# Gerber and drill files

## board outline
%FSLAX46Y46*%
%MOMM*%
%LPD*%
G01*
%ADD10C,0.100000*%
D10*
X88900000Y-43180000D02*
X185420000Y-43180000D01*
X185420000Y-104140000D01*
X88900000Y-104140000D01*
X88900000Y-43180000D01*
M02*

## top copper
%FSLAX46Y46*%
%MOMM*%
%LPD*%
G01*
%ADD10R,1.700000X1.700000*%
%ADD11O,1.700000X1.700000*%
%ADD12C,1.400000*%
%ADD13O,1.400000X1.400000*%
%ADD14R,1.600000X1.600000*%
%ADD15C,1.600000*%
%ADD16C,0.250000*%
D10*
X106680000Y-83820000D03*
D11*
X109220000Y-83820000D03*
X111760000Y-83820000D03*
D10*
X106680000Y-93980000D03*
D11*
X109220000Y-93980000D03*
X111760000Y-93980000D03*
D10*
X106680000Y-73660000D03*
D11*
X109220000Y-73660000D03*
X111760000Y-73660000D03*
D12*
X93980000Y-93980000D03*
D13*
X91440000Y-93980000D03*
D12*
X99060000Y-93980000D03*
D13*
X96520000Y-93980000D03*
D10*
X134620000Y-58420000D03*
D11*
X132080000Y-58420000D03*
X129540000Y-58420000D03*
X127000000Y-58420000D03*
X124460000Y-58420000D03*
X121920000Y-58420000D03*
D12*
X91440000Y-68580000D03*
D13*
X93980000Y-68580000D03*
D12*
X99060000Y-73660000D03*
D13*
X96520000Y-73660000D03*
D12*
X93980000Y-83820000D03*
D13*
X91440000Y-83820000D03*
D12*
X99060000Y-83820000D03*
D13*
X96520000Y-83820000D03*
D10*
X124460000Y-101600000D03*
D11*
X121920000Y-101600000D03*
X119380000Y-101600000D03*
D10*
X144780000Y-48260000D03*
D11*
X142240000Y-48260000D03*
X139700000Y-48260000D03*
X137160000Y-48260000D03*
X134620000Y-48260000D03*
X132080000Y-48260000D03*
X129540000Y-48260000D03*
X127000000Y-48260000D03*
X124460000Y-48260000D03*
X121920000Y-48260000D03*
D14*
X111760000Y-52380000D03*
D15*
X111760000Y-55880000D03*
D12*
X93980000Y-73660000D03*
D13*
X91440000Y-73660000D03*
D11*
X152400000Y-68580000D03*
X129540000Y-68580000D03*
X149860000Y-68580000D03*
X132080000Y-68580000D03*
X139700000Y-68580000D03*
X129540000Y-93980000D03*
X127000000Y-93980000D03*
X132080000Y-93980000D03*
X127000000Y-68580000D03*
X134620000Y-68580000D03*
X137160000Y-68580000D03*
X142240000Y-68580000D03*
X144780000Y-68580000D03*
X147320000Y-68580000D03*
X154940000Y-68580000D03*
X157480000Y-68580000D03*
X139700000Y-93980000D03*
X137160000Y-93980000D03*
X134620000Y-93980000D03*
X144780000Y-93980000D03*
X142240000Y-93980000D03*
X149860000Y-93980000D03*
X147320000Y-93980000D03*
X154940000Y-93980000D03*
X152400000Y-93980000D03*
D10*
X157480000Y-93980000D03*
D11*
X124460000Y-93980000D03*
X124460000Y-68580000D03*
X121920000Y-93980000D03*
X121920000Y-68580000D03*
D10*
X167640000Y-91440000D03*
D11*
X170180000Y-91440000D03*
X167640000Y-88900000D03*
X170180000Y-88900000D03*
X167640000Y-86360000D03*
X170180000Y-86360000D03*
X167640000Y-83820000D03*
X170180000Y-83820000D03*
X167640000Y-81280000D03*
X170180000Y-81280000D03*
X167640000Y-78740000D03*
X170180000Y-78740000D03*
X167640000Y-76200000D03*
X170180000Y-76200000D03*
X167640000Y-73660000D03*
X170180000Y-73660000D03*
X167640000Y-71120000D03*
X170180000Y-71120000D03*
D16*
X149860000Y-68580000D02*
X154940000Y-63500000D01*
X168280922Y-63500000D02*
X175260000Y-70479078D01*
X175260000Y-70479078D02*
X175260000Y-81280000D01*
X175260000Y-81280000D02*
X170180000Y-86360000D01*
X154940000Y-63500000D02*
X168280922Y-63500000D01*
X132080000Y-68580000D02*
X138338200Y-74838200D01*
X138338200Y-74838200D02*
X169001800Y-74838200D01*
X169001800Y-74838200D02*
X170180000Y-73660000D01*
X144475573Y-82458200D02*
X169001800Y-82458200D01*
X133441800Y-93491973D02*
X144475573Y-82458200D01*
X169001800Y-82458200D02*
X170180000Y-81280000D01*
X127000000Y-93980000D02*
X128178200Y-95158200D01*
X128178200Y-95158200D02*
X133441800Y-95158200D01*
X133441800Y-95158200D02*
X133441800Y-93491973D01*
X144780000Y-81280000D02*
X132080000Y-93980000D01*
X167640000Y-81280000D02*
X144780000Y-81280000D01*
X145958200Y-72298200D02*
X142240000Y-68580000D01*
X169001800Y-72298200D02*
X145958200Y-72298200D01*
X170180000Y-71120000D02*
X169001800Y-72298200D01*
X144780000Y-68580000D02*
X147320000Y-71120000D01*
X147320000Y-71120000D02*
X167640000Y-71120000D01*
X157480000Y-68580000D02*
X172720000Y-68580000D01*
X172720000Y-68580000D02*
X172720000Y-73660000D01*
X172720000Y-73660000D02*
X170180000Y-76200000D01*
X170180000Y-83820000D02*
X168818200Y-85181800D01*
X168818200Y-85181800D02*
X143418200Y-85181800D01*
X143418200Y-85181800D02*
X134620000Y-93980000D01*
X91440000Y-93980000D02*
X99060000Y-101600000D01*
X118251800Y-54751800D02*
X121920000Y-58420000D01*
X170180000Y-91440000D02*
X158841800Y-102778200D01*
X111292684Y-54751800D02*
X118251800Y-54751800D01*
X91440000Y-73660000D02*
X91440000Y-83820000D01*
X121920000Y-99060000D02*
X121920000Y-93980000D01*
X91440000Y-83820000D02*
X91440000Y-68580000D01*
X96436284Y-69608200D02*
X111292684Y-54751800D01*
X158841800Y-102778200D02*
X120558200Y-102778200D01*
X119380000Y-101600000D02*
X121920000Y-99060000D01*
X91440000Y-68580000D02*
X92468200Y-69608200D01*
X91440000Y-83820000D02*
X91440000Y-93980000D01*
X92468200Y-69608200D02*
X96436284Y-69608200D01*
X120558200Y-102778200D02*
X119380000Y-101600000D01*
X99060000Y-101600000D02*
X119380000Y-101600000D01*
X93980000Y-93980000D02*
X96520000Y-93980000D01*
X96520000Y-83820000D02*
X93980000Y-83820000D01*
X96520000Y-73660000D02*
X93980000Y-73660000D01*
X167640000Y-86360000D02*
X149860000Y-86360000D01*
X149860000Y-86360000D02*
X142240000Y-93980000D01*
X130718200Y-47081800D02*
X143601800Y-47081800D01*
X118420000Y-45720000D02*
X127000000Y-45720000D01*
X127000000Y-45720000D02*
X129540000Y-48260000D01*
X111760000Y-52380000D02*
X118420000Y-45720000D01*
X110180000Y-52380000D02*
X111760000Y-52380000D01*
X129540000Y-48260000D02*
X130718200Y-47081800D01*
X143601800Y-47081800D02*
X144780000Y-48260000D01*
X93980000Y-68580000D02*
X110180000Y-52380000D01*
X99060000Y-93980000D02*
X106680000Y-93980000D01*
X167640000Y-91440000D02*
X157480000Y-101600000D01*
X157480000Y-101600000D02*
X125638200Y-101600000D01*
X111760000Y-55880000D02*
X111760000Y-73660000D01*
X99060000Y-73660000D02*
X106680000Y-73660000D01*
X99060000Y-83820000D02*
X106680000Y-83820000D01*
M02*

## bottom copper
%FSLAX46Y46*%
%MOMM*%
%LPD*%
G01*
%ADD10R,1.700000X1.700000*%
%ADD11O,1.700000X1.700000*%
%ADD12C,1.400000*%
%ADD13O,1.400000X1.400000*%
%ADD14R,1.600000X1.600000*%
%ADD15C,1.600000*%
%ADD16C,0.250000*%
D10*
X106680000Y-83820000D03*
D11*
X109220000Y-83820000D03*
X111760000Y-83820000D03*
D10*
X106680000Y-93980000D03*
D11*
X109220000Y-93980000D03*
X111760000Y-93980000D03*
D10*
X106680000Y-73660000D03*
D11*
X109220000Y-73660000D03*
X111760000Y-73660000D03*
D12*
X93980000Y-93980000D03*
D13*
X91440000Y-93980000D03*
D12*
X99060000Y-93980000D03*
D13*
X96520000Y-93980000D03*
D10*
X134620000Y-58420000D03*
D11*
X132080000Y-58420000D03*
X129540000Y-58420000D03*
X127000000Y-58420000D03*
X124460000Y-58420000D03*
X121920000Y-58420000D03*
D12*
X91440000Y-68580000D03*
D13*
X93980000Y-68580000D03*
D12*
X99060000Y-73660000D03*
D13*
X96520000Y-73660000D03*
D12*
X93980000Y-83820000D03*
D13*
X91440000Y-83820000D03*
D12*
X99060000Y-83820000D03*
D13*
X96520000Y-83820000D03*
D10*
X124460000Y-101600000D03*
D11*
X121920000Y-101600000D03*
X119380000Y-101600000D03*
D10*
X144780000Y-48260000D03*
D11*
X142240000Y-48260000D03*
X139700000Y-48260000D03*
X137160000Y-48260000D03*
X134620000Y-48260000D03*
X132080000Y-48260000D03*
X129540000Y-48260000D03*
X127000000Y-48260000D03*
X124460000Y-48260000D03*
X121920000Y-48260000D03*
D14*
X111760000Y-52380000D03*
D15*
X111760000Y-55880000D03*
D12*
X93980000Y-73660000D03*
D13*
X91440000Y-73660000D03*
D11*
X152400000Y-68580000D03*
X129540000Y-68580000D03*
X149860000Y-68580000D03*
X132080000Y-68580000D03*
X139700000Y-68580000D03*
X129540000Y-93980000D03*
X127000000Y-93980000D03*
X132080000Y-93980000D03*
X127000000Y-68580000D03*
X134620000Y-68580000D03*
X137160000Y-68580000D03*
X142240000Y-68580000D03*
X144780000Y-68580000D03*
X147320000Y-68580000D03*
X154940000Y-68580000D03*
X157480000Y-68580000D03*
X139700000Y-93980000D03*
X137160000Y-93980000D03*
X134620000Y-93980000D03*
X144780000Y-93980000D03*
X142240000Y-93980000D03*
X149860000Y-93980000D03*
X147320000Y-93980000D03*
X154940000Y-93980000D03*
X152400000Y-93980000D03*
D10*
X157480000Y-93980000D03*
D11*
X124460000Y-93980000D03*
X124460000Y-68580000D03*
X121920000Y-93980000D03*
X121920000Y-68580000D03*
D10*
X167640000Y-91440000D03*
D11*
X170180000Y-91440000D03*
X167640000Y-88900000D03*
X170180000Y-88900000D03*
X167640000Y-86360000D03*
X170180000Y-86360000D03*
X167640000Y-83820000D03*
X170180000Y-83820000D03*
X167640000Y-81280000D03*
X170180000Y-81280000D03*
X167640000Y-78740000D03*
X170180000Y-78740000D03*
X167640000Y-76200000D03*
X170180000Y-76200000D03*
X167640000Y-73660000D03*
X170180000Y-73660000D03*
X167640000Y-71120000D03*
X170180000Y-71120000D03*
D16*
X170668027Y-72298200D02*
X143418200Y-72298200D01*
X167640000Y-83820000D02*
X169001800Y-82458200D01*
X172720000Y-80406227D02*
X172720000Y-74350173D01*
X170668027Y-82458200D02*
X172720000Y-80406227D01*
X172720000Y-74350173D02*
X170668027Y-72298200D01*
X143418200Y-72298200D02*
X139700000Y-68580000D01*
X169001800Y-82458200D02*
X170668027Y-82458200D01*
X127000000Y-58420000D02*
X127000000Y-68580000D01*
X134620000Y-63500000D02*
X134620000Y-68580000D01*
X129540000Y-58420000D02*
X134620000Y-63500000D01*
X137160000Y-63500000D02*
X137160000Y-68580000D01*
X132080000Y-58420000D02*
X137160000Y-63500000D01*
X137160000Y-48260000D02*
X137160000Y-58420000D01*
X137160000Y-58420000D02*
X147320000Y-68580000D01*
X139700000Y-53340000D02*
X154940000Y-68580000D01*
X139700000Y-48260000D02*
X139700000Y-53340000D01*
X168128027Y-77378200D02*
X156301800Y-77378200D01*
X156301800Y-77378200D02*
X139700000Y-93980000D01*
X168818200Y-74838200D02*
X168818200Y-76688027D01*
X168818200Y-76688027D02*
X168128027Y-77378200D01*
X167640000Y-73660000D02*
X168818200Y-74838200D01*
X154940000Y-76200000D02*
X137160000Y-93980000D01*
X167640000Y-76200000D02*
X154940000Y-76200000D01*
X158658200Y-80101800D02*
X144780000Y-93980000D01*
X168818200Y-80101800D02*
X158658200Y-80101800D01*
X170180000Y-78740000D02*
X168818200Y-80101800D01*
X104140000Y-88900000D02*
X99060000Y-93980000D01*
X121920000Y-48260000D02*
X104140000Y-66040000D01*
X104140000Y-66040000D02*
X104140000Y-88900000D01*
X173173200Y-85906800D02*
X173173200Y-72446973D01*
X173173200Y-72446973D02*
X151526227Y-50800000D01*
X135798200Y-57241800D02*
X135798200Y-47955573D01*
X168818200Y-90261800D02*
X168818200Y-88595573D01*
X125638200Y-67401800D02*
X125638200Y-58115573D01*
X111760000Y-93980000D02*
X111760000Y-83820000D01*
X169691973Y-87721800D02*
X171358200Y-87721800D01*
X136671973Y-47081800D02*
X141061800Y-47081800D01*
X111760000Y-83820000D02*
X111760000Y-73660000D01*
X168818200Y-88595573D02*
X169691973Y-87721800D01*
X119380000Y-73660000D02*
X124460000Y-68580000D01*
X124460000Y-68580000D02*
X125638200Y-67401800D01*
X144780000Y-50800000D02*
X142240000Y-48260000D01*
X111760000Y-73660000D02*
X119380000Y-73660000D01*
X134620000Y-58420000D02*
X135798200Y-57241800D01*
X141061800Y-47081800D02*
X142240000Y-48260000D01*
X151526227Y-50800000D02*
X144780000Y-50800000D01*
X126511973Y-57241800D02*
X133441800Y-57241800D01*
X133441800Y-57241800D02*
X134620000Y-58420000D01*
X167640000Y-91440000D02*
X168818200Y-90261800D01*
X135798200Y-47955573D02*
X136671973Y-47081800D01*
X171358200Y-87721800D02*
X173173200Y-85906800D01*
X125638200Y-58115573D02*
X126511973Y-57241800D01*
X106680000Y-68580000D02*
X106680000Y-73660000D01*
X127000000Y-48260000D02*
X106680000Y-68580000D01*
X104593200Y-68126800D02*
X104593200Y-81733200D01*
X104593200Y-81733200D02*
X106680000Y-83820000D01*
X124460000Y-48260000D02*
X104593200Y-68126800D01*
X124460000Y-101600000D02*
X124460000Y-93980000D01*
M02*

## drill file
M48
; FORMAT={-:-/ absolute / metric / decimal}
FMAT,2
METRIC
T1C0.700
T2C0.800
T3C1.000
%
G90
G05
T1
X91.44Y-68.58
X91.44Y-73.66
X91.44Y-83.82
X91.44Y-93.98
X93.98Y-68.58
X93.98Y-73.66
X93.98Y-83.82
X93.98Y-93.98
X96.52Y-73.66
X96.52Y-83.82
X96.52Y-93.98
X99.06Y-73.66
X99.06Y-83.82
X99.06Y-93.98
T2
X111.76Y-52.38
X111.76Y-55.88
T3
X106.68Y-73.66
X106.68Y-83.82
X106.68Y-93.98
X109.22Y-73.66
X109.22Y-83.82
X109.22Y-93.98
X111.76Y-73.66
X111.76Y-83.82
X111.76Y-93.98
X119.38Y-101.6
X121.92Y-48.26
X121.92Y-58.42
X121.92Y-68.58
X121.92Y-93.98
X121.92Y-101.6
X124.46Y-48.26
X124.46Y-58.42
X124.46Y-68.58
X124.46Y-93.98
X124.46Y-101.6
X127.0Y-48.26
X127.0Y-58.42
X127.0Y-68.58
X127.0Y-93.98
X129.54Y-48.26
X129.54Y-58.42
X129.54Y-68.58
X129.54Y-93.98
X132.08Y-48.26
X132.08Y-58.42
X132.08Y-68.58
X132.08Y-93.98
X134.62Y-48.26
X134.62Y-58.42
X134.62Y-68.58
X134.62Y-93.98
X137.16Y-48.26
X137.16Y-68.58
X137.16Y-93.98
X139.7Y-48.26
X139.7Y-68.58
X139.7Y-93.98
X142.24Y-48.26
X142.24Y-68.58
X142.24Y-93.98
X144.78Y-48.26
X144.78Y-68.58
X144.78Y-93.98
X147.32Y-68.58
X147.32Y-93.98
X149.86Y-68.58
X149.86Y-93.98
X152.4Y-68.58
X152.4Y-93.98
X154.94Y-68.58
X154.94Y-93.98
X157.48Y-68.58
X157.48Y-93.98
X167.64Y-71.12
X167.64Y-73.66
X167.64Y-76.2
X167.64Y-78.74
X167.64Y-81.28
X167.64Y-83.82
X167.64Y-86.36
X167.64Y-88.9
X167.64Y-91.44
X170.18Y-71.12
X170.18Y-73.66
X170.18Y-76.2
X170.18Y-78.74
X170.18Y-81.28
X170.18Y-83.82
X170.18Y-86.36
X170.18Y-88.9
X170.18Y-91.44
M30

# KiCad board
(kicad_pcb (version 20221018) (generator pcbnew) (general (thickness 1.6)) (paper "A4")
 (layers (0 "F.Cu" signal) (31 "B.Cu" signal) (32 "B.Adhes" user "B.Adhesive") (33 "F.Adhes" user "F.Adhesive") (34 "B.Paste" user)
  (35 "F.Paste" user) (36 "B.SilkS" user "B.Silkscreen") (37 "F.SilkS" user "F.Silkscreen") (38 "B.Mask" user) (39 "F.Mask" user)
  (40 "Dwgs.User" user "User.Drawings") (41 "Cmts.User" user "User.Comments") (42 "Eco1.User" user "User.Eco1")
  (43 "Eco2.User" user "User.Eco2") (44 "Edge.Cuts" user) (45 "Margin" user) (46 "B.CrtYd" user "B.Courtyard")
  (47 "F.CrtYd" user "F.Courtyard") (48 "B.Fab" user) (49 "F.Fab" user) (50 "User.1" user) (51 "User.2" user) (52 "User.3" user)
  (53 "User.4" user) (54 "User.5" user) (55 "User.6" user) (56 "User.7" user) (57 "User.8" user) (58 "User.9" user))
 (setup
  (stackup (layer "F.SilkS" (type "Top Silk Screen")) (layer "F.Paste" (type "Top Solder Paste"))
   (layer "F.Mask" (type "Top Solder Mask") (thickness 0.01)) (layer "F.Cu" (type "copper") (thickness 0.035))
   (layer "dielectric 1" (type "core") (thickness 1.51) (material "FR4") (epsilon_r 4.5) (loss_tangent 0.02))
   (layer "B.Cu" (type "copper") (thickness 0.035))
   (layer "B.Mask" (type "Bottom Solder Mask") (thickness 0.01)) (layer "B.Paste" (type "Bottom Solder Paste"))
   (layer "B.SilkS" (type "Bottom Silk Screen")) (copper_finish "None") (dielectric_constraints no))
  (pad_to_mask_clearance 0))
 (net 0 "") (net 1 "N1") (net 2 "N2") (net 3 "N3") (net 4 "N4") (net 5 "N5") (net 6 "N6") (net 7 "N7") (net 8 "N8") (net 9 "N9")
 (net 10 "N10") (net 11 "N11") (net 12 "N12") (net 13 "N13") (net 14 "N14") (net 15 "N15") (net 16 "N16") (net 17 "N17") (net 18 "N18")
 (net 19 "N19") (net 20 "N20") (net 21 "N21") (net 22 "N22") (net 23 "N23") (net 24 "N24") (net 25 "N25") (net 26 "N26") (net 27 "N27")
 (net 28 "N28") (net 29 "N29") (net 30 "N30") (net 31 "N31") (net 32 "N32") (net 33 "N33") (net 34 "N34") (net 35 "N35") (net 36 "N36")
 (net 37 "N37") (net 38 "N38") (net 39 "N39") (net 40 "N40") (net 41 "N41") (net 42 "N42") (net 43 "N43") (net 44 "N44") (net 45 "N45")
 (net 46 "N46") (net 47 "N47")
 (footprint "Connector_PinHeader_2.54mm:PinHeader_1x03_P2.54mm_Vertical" (layer "F.Cu") (at 106.68 83.82 90)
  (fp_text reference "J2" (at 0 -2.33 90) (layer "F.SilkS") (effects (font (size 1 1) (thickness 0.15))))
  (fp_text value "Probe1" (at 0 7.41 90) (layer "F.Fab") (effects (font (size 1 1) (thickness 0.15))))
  (pad "1" thru_hole rect (at 0 0 90) (size 1.7 1.7) (drill 1) (layers "*.Cu" "*.Mask") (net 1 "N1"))
  (pad "2" thru_hole oval (at 0 2.54 90) (size 1.7 1.7) (drill 1) (layers "*.Cu" "*.Mask") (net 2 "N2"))
  (pad "3" thru_hole oval (at 0 5.08 90) (size 1.7 1.7) (drill 1) (layers "*.Cu" "*.Mask") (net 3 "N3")))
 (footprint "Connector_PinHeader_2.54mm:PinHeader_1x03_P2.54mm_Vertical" (layer "F.Cu") (at 106.68 93.98 90)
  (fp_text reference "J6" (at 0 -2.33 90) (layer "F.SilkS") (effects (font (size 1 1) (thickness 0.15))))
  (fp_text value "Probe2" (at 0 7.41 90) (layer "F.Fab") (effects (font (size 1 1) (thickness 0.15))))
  (pad "1" thru_hole rect (at 0 0 90) (size 1.7 1.7) (drill 1) (layers "*.Cu" "*.Mask") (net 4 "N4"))
  (pad "2" thru_hole oval (at 0 2.54 90) (size 1.7 1.7) (drill 1) (layers "*.Cu" "*.Mask") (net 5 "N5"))
  (pad "3" thru_hole oval (at 0 5.08 90) (size 1.7 1.7) (drill 1) (layers "*.Cu" "*.Mask") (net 3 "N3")))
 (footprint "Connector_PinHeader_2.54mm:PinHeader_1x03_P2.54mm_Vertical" (layer "F.Cu") (at 106.68 73.66 90)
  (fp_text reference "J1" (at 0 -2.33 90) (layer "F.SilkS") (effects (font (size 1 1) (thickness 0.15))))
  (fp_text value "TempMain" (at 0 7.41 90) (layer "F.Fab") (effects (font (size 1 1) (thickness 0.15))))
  (pad "1" thru_hole rect (at 0 0 90) (size 1.7 1.7) (drill 1) (layers "*.Cu" "*.Mask") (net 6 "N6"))
  (pad "2" thru_hole oval (at 0 2.54 90) (size 1.7 1.7) (drill 1) (layers "*.Cu" "*.Mask") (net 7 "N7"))
  (pad "3" thru_hole oval (at 0 5.08 90) (size 1.7 1.7) (drill 1) (layers "*.Cu" "*.Mask") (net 3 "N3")))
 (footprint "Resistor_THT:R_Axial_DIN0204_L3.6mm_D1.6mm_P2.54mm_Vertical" (layer "F.Cu") (at 93.98 93.98 180)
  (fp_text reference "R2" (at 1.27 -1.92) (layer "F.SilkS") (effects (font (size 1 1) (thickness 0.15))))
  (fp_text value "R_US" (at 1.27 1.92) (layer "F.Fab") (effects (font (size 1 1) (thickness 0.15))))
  (pad "1" thru_hole circle (at 0 0 180) (size 1.4 1.4) (drill 0.7) (layers "*.Cu" "*.Mask") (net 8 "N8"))
  (pad "2" thru_hole oval (at 2.54 0 180) (size 1.4 1.4) (drill 0.7) (layers "*.Cu" "*.Mask") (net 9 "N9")))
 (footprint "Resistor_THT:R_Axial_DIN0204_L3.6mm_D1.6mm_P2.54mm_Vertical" (layer "F.Cu") (at 99.06 93.98 180)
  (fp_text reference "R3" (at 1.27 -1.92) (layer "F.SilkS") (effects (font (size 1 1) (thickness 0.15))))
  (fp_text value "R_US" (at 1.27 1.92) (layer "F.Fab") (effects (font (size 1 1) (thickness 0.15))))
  (pad "1" thru_hole circle (at 0 0 180) (size 1.4 1.4) (drill 0.7) (layers "*.Cu" "*.Mask") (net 4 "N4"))
  (pad "2" thru_hole oval (at 2.54 0 180) (size 1.4 1.4) (drill 0.7) (layers "*.Cu" "*.Mask") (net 8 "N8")))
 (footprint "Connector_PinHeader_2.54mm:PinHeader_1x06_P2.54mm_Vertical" (layer "F.Cu") (at 134.62 58.42 -90)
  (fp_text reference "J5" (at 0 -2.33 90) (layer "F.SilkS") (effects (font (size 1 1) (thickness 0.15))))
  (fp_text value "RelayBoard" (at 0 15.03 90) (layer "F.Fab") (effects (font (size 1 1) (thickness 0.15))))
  (pad "1" thru_hole rect (at 0 0 270) (size 1.7 1.7) (drill 1) (layers "*.Cu" "*.Mask") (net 3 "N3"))
  (pad "2" thru_hole oval (at 0 2.54 270) (size 1.7 1.7) (drill 1) (layers "*.Cu" "*.Mask") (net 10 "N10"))
  (pad "3" thru_hole oval (at 0 5.08 270) (size 1.7 1.7) (drill 1) (layers "*.Cu" "*.Mask") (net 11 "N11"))
  (pad "4" thru_hole oval (at 0 7.62 270) (size 1.7 1.7) (drill 1) (layers "*.Cu" "*.Mask") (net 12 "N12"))
  (pad "5" thru_hole oval (at 0 10.16 270) (size 1.7 1.7) (drill 1) (layers "*.Cu" "*.Mask") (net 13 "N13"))
  (pad "6" thru_hole oval (at 0 12.7 270) (size 1.7 1.7) (drill 1) (layers "*.Cu" "*.Mask") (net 9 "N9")))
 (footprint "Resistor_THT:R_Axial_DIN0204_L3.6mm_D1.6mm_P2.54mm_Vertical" (layer "F.Cu") (at 91.44 68.58)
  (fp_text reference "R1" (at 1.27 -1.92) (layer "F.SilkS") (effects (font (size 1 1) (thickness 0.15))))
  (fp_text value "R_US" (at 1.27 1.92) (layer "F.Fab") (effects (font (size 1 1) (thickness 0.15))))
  (pad "1" thru_hole circle (at 0 0) (size 1.4 1.4) (drill 0.7) (layers "*.Cu" "*.Mask") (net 9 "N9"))
  (pad "2" thru_hole oval (at 2.54 0) (size 1.4 1.4) (drill 0.7) (layers "*.Cu" "*.Mask") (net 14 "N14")))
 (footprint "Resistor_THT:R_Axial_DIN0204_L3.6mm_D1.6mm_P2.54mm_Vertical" (layer "F.Cu") (at 99.06 73.66 180)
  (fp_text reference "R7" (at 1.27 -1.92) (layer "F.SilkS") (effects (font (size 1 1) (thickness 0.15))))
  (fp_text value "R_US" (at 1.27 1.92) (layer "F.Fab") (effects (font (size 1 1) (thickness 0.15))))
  (pad "1" thru_hole circle (at 0 0 180) (size 1.4 1.4) (drill 0.7) (layers "*.Cu" "*.Mask") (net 6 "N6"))
  (pad "2" thru_hole oval (at 2.54 0 180) (size 1.4 1.4) (drill 0.7) (layers "*.Cu" "*.Mask") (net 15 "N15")))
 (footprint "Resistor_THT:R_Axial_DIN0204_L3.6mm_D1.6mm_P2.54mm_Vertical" (layer "F.Cu") (at 93.98 83.82 180)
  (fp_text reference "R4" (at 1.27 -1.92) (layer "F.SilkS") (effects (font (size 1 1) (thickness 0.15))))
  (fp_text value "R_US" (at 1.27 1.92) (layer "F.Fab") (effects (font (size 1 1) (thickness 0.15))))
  (pad "1" thru_hole circle (at 0 0 180) (size 1.4 1.4) (drill 0.7) (layers "*.Cu" "*.Mask") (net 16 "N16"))
  (pad "2" thru_hole oval (at 2.54 0 180) (size 1.4 1.4) (drill 0.7) (layers "*.Cu" "*.Mask") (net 9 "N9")))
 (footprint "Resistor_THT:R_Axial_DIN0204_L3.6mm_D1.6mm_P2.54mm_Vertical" (layer "F.Cu") (at 99.06 83.82 180)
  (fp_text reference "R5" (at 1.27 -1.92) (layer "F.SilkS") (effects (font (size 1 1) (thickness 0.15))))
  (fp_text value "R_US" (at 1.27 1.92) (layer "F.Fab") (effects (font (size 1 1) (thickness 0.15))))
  (pad "1" thru_hole circle (at 0 0 180) (size 1.4 1.4) (drill 0.7) (layers "*.Cu" "*.Mask") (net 1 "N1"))
  (pad "2" thru_hole oval (at 2.54 0 180) (size 1.4 1.4) (drill 0.7) (layers "*.Cu" "*.Mask") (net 16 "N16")))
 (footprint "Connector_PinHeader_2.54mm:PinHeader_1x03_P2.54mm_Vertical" (layer "F.Cu") (at 124.46 101.6 -90)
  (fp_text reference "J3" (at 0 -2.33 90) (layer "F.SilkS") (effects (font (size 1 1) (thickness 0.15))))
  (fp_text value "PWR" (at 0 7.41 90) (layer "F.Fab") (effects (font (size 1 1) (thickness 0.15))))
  (pad "1" thru_hole rect (at 0 0 270) (size 1.7 1.7) (drill 1) (layers "*.Cu" "*.Mask") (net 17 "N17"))
  (pad "2" thru_hole oval (at 0 2.54 270) (size 1.7 1.7) (drill 1) (layers "*.Cu" "*.Mask") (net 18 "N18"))
  (pad "3" thru_hole oval (at 0 5.08 270) (size 1.7 1.7) (drill 1) (layers "*.Cu" "*.Mask") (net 9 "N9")))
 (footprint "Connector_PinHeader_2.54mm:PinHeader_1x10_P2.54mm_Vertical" (layer "F.Cu") (at 144.78 48.26 -90)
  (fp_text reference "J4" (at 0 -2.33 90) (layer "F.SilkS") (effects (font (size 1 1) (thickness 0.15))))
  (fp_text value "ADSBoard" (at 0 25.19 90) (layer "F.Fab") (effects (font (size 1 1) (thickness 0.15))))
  (pad "1" thru_hole rect (at 0 0 270) (size 1.7 1.7) (drill 1) (layers "*.Cu" "*.Mask") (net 14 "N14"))
  (pad "2" thru_hole oval (at 0 2.54 270) (size 1.7 1.7) (drill 1) (layers "*.Cu" "*.Mask") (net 3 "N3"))
  (pad "3" thru_hole oval (at 0 5.08 270) (size 1.7 1.7) (drill 1) (layers "*.Cu" "*.Mask") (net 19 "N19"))
  (pad "4" thru_hole oval (at 0 7.62 270) (size 1.7 1.7) (drill 1) (layers "*.Cu" "*.Mask") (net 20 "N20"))
  (pad "5" thru_hole oval (at 0 10.16 270) (size 1.7 1.7) (drill 1) (layers "*.Cu" "*.Mask") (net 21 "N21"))
  (pad "6" thru_hole oval (at 0 12.7 270) (size 1.7 1.7) (drill 1) (layers "*.Cu" "*.Mask") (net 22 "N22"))
  (pad "7" thru_hole oval (at 0 15.24 270) (size 1.7 1.7) (drill 1) (layers "*.Cu" "*.Mask") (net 14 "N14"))
  (pad "8" thru_hole oval (at 0 17.78 270) (size 1.7 1.7) (drill 1) (layers "*.Cu" "*.Mask") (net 6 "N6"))
  (pad "9" thru_hole oval (at 0 20.32 270) (size 1.7 1.7) (drill 1) (layers "*.Cu" "*.Mask") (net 1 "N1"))
  (pad "10" thru_hole oval (at 0 22.86 270) (size 1.7 1.7) (drill 1) (layers "*.Cu" "*.Mask") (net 4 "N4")))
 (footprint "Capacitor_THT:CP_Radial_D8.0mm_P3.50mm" (layer "F.Cu") (at 111.76 52.38 -90)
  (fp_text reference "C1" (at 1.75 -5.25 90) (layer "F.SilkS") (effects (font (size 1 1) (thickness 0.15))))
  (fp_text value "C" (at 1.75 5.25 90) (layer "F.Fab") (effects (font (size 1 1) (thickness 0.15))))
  (pad "1" thru_hole rect (at 0 0 270) (size 1.6 1.6) (drill 0.8) (layers "*.Cu" "*.Mask") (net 14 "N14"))
  (pad "2" thru_hole circle (at 3.5 0 270) (size 1.6 1.6) (drill 0.8) (layers "*.Cu" "*.Mask") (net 3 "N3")))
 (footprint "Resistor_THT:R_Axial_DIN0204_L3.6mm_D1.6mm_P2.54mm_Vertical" (layer "F.Cu") (at 93.98 73.66 180)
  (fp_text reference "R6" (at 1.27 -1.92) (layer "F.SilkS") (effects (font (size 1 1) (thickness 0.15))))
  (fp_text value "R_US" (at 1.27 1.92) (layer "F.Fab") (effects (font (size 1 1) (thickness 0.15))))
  (pad "1" thru_hole circle (at 0 0 180) (size 1.4 1.4) (drill 0.7) (layers "*.Cu" "*.Mask") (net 15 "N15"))
  (pad "2" thru_hole oval (at 2.54 0 180) (size 1.4 1.4) (drill 0.7) (layers "*.Cu" "*.Mask") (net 9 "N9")))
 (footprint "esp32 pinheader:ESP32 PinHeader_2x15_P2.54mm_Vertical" (layer "B.Cu") (at 157.48 93.98 90)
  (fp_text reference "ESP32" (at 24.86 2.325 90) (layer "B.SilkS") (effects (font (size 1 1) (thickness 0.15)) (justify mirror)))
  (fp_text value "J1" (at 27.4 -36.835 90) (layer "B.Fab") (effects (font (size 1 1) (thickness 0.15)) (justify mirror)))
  (pad "1" thru_hole oval (at 25.4 -5.08 90) (size 1.7 1.7) (drill 1) (layers "*.Cu" "*.Mask") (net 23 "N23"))
  (pad "2" thru_hole oval (at 25.4 -27.94 90) (size 1.7 1.7) (drill 1) (layers "*.Cu" "*.Mask") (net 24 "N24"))
  (pad "3" thru_hole oval (at 25.4 -7.62 90) (size 1.7 1.7) (drill 1) (layers "*.Cu" "*.Mask") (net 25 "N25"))
  (pad "4" thru_hole oval (at 25.4 -25.4 90) (size 1.7 1.7) (drill 1) (layers "*.Cu" "*.Mask") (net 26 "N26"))
  (pad "5" thru_hole oval (at 25.4 -17.78 90) (size 1.7 1.7) (drill 1) (layers "*.Cu" "*.Mask") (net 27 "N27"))
  (pad "12" thru_hole oval (at 0 -27.94 90) (size 1.7 1.7) (drill 1) (layers "*.Cu" "*.Mask") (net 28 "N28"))
  (pad "13" thru_hole oval (at 0 -30.48 90) (size 1.7 1.7) (drill 1) (layers "*.Cu" "*.Mask") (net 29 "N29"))
  (pad "14" thru_hole oval (at 0 -25.4 90) (size 1.7 1.7) (drill 1) (layers "*.Cu" "*.Mask") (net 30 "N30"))
  (pad "15" thru_hole oval (at 25.4 -30.48 90) (size 1.7 1.7) (drill 1) (layers "*.Cu" "*.Mask") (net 12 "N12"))
  (pad "16" thru_hole oval (at 25.4 -22.86 90) (size 1.7 1.7) (drill 1) (layers "*.Cu" "*.Mask") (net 11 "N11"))
  (pad "17" thru_hole oval (at 25.4 -20.32 90) (size 1.7 1.7) (drill 1) (layers "*.Cu" "*.Mask") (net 10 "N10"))
  (pad "18" thru_hole oval (at 25.4 -15.24 90) (size 1.7 1.7) (drill 1) (layers "*.Cu" "*.Mask") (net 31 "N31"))
  (pad "19" thru_hole oval (at 25.4 -12.7 90) (size 1.7 1.7) (drill 1) (layers "*.Cu" "*.Mask") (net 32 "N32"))
  (pad "21" thru_hole oval (at 25.4 -10.16 90) (size 1.7 1.7) (drill 1) (layers "*.Cu" "*.Mask") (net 20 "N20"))
  (pad "22" thru_hole oval (at 25.4 -2.54 90) (size 1.7 1.7) (drill 1) (layers "*.Cu" "*.Mask") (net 19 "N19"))
  (pad "23" thru_hole oval (at 25.4 0 90) (size 1.7 1.7) (drill 1) (layers "*.Cu" "*.Mask") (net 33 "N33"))
  (pad "25" thru_hole oval (at 0 -17.78 90) (size 1.7 1.7) (drill 1) (layers "*.Cu" "*.Mask") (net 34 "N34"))
  (pad "26" thru_hole oval (at 0 -20.32 90) (size 1.7 1.7) (drill 1) (layers "*.Cu" "*.Mask") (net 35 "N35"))
  (pad "27" thru_hole oval (at 0 -22.86 90) (size 1.7 1.7) (drill 1) (layers "*.Cu" "*.Mask") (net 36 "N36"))
  (pad "32" thru_hole oval (at 0 -12.7 90) (size 1.7 1.7) (drill 1) (layers "*.Cu" "*.Mask") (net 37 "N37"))
  (pad "33" thru_hole oval (at 0 -15.24 90) (size 1.7 1.7) (drill 1) (layers "*.Cu" "*.Mask") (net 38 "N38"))
  (pad "34" thru_hole oval (at 0 -7.62 90) (size 1.7 1.7) (drill 1) (layers "*.Cu" "*.Mask") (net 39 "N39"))
  (pad "35" thru_hole oval (at 0 -10.16 90) (size 1.7 1.7) (drill 1) (layers "*.Cu" "*.Mask") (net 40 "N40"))
  (pad "36" thru_hole oval (at 0 -2.54 90) (size 1.7 1.7) (drill 1) (layers "*.Cu" "*.Mask") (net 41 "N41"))
  (pad "39" thru_hole oval (at 0 -5.08 90) (size 1.7 1.7) (drill 1) (layers "*.Cu" "*.Mask") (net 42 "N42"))
  (pad "60" thru_hole rect (at 0 0 90) (size 1.7 1.7) (drill 1) (layers "*.Cu" "*.Mask") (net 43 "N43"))
  (pad "61" thru_hole oval (at 0 -33.02 90) (size 1.7 1.7) (drill 1) (layers "*.Cu" "*.Mask") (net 17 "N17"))
  (pad "62" thru_hole oval (at 25.4 -33.02 90) (size 1.7 1.7) (drill 1) (layers "*.Cu" "*.Mask") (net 3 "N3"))
  (pad "63" thru_hole oval (at 0 -35.56 90) (size 1.7 1.7) (drill 1) (layers "*.Cu" "*.Mask") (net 9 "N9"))
  (pad "64" thru_hole oval (at 25.4 -35.56 90) (size 1.7 1.7) (drill 1) (layers "*.Cu" "*.Mask") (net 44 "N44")))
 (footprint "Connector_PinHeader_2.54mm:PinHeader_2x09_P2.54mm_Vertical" (layer "B.Cu") (at 167.64 91.44)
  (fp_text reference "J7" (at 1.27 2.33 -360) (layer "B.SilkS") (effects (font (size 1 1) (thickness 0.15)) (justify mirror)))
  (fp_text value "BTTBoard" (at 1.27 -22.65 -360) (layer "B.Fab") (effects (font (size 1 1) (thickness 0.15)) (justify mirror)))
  (pad "1" thru_hole rect (at 0 0) (size 1.7 1.7) (drill 1) (layers "*.Cu" "*.Mask") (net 3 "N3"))
  (pad "2" thru_hole oval (at 2.54 0) (size 1.7 1.7) (drill 1) (layers "*.Cu" "*.Mask") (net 9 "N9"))
  (pad "3" thru_hole oval (at 0 -2.54) (size 1.7 1.7) (drill 1) (layers "*.Cu" "*.Mask") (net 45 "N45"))
  (pad "4" thru_hole oval (at 2.54 -2.54) (size 1.7 1.7) (drill 1) (layers "*.Cu" "*.Mask") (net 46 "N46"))
  (pad "5" thru_hole oval (at 0 -5.08) (size 1.7 1.7) (drill 1) (layers "*.Cu" "*.Mask") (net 38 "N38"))
  (pad "6" thru_hole oval (at 2.54 -5.08) (size 1.7 1.7) (drill 1) (layers "*.Cu" "*.Mask") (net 25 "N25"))
  (pad "7" thru_hole oval (at 0 -7.62) (size 1.7 1.7) (drill 1) (layers "*.Cu" "*.Mask") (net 27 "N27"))
  (pad "8" thru_hole oval (at 2.54 -7.62) (size 1.7 1.7) (drill 1) (layers "*.Cu" "*.Mask") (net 36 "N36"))
  (pad "9" thru_hole oval (at 0 -10.16) (size 1.7 1.7) (drill 1) (layers "*.Cu" "*.Mask") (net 30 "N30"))
  (pad "10" thru_hole oval (at 2.54 -10.16) (size 1.7 1.7) (drill 1) (layers "*.Cu" "*.Mask") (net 29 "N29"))
  (pad "11" thru_hole oval (at 0 -12.7) (size 1.7 1.7) (drill 1) (layers "*.Cu" "*.Mask") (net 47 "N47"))
  (pad "12" thru_hole oval (at 2.54 -12.7) (size 1.7 1.7) (drill 1) (layers "*.Cu" "*.Mask") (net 37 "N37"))
  (pad "13" thru_hole oval (at 0 -15.24) (size 1.7 1.7) (drill 1) (layers "*.Cu" "*.Mask") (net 35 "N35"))
  (pad "14" thru_hole oval (at 2.54 -15.24) (size 1.7 1.7) (drill 1) (layers "*.Cu" "*.Mask") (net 33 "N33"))
  (pad "15" thru_hole oval (at 0 -17.78) (size 1.7 1.7) (drill 1) (layers "*.Cu" "*.Mask") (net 34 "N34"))
  (pad "16" thru_hole oval (at 2.54 -17.78) (size 1.7 1.7) (drill 1) (layers "*.Cu" "*.Mask") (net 26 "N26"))
  (pad "17" thru_hole oval (at 0 -20.32) (size 1.7 1.7) (drill 1) (layers "*.Cu" "*.Mask") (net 32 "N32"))
  (pad "18" thru_hole oval (at 2.54 -20.32) (size 1.7 1.7) (drill 1) (layers "*.Cu" "*.Mask") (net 31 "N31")))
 (gr_rect (start 88.9 43.18) (end 185.42 104.14) (stroke (width 0.1) (type default)) (fill none) (layer "Edge.Cuts"))
 (segment (start 149.86 68.58) (end 154.94 63.5) (width 0.25) (layer "F.Cu") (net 25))
 (segment (start 168.280922 63.5) (end 175.26 70.479078) (width 0.25) (layer "F.Cu") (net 25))
 (segment (start 175.26 70.479078) (end 175.26 81.28) (width 0.25) (layer "F.Cu") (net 25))
 (segment (start 175.26 81.28) (end 170.18 86.36) (width 0.25) (layer "F.Cu") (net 25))
 (segment (start 154.94 63.5) (end 168.280922 63.5) (width 0.25) (layer "F.Cu") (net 25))
 (segment (start 132.08 68.58) (end 138.3382 74.8382) (width 0.25) (layer "F.Cu") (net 26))
 (segment (start 138.3382 74.8382) (end 169.0018 74.8382) (width 0.25) (layer "F.Cu") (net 26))
 (segment (start 169.0018 74.8382) (end 170.18 73.66) (width 0.25) (layer "F.Cu") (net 26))
 (segment (start 170.668027 72.2982) (end 143.4182 72.2982) (width 0.25) (layer "B.Cu") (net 27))
 (segment (start 167.64 83.82) (end 169.0018 82.4582) (width 0.25) (layer "B.Cu") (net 27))
 (segment (start 172.72 80.406227) (end 172.72 74.350173) (width 0.25) (layer "B.Cu") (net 27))
 (segment (start 170.668027 82.4582) (end 172.72 80.406227) (width 0.25) (layer "B.Cu") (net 27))
 (segment (start 172.72 74.350173) (end 170.668027 72.2982) (width 0.25) (layer "B.Cu") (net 27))
 (segment (start 143.4182 72.2982) (end 139.7 68.58) (width 0.25) (layer "B.Cu") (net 27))
 (segment (start 169.0018 82.4582) (end 170.668027 82.4582) (width 0.25) (layer "B.Cu") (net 27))
 (segment (start 144.475573 82.4582) (end 169.0018 82.4582) (width 0.25) (layer "F.Cu") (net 29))
 (segment (start 133.4418 93.491973) (end 144.475573 82.4582) (width 0.25) (layer "F.Cu") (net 29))
 (segment (start 169.0018 82.4582) (end 170.18 81.28) (width 0.25) (layer "F.Cu") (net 29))
 (segment (start 127 93.98) (end 128.1782 95.1582) (width 0.25) (layer "F.Cu") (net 29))
 (segment (start 128.1782 95.1582) (end 133.4418 95.1582) (width 0.25) (layer "F.Cu") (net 29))
 (segment (start 133.4418 95.1582) (end 133.4418 93.491973) (width 0.25) (layer "F.Cu") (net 29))
 (segment (start 144.78 81.28) (end 132.08 93.98) (width 0.25) (layer "F.Cu") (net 30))
 (segment (start 167.64 81.28) (end 144.78 81.28) (width 0.25) (layer "F.Cu") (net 30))
 (segment (start 127 58.42) (end 127 68.58) (width 0.25) (layer "B.Cu") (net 12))
 (segment (start 134.62 63.5) (end 134.62 68.58) (width 0.25) (layer "B.Cu") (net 11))
 (segment (start 129.54 58.42) (end 134.62 63.5) (width 0.25) (layer "B.Cu") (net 11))
 (segment (start 137.16 63.5) (end 137.16 68.58) (width 0.25) (layer "B.Cu") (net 10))
 (segment (start 132.08 58.42) (end 137.16 63.5) (width 0.25) (layer "B.Cu") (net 10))
 (segment (start 145.9582 72.2982) (end 142.24 68.58) (width 0.25) (layer "F.Cu") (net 31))
 (segment (start 169.0018 72.2982) (end 145.9582 72.2982) (width 0.25) (layer "F.Cu") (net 31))
 (segment (start 170.18 71.12) (end 169.0018 72.2982) (width 0.25) (layer "F.Cu") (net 31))
 (segment (start 144.78 68.58) (end 147.32 71.12) (width 0.25) (layer "F.Cu") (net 32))
 (segment (start 147.32 71.12) (end 167.64 71.12) (width 0.25) (layer "F.Cu") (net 32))
 (segment (start 137.16 48.26) (end 137.16 58.42) (width 0.25) (layer "B.Cu") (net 20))
 (segment (start 137.16 58.42) (end 147.32 68.58) (width 0.25) (layer "B.Cu") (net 20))
 (segment (start 139.7 53.34) (end 154.94 68.58) (width 0.25) (layer "B.Cu") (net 19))
 (segment (start 139.7 48.26) (end 139.7 53.34) (width 0.25) (layer "B.Cu") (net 19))
 (segment (start 157.48 68.58) (end 172.72 68.58) (width 0.25) (layer "F.Cu") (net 33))
 (segment (start 172.72 68.58) (end 172.72 73.66) (width 0.25) (layer "F.Cu") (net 33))
 (segment (start 172.72 73.66) (end 170.18 76.2) (width 0.25) (layer "F.Cu") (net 33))
 (segment (start 168.128027 77.3782) (end 156.3018 77.3782) (width 0.25) (layer "B.Cu") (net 34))
 (segment (start 156.3018 77.3782) (end 139.7 93.98) (width 0.25) (layer "B.Cu") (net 34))
 (segment (start 168.8182 74.8382) (end 168.8182 76.688027) (width 0.25) (layer "B.Cu") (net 34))
 (segment (start 168.8182 76.688027) (end 168.128027 77.3782) (width 0.25) (layer "B.Cu") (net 34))
 (segment (start 167.64 73.66) (end 168.8182 74.8382) (width 0.25) (layer "B.Cu") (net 34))
 (segment (start 154.94 76.2) (end 137.16 93.98) (width 0.25) (layer "B.Cu") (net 35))
 (segment (start 167.64 76.2) (end 154.94 76.2) (width 0.25) (layer "B.Cu") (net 35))
 (segment (start 170.18 83.82) (end 168.8182 85.1818) (width 0.25) (layer "F.Cu") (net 36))
 (segment (start 168.8182 85.1818) (end 143.4182 85.1818) (width 0.25) (layer "F.Cu") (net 36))
 (segment (start 143.4182 85.1818) (end 134.62 93.98) (width 0.25) (layer "F.Cu") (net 36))
 (segment (start 91.44 93.98) (end 99.06 101.6) (width 0.25) (layer "F.Cu") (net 9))
 (segment (start 118.2518 54.7518) (end 121.92 58.42) (width 0.25) (layer "F.Cu") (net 9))
 (segment (start 170.18 91.44) (end 158.8418 102.7782) (width 0.25) (layer "F.Cu") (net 9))
 (segment (start 111.292684 54.7518) (end 118.2518 54.7518) (width 0.25) (layer "F.Cu") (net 9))
 (segment (start 91.44 73.66) (end 91.44 83.82) (width 0.25) (layer "F.Cu") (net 9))
 (segment (start 121.92 99.06) (end 121.92 93.98) (width 0.25) (layer "F.Cu") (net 9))
 (segment (start 91.44 83.82) (end 91.44 68.58) (width 0.25) (layer "F.Cu") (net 9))
 (segment (start 96.436284 69.6082) (end 111.292684 54.7518) (width 0.25) (layer "F.Cu") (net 9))
 (segment (start 158.8418 102.7782) (end 120.5582 102.7782) (width 0.25) (layer "F.Cu") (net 9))
 (segment (start 119.38 101.6) (end 121.92 99.06) (width 0.25) (layer "F.Cu") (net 9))
 (segment (start 91.44 68.58) (end 92.4682 69.6082) (width 0.25) (layer "F.Cu") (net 9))
 (segment (start 91.44 83.82) (end 91.44 93.98) (width 0.25) (layer "F.Cu") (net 9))
 (segment (start 92.4682 69.6082) (end 96.436284 69.6082) (width 0.25) (layer "F.Cu") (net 9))
 (segment (start 120.5582 102.7782) (end 119.38 101.6) (width 0.25) (layer "F.Cu") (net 9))
 (segment (start 99.06 101.6) (end 119.38 101.6) (width 0.25) (layer "F.Cu") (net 9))
 (segment (start 93.98 93.98) (end 96.52 93.98) (width 0.25) (layer "F.Cu") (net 8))
 (segment (start 96.52 83.82) (end 93.98 83.82) (width 0.25) (layer "F.Cu") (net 16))
 (segment (start 96.52 73.66) (end 93.98 73.66) (width 0.25) (layer "F.Cu") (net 15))
 (segment (start 167.64 86.36) (end 149.86 86.36) (width 0.25) (layer "F.Cu") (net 38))
 (segment (start 149.86 86.36) (end 142.24 93.98) (width 0.25) (layer "F.Cu") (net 38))
 (segment (start 158.6582 80.1018) (end 144.78 93.98) (width 0.25) (layer "B.Cu") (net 37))
 (segment (start 168.8182 80.1018) (end 158.6582 80.1018) (width 0.25) (layer "B.Cu") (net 37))
 (segment (start 170.18 78.74) (end 168.8182 80.1018) (width 0.25) (layer "B.Cu") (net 37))
 (segment (start 130.7182 47.0818) (end 143.6018 47.0818) (width 0.25) (layer "F.Cu") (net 14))
 (segment (start 118.42 45.72) (end 127 45.72) (width 0.25) (layer "F.Cu") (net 14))
 (segment (start 127 45.72) (end 129.54 48.26) (width 0.25) (layer "F.Cu") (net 14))
 (segment (start 111.76 52.38) (end 118.42 45.72) (width 0.25) (layer "F.Cu") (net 14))
 (segment (start 110.18 52.38) (end 111.76 52.38) (width 0.25) (layer "F.Cu") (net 14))
 (segment (start 129.54 48.26) (end 130.7182 47.0818) (width 0.25) (layer "F.Cu") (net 14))
 (segment (start 143.6018 47.0818) (end 144.78 48.26) (width 0.25) (layer "F.Cu") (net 14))
 (segment (start 93.98 68.58) (end 110.18 52.38) (width 0.25) (layer "F.Cu") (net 14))
 (segment (start 99.06 93.98) (end 106.68 93.98) (width 0.25) (layer "F.Cu") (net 4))
 (segment (start 104.14 88.9) (end 99.06 93.98) (width 0.25) (layer "B.Cu") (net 4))
 (segment (start 121.92 48.26) (end 104.14 66.04) (width 0.25) (layer "B.Cu") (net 4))
 (segment (start 104.14 66.04) (end 104.14 88.9) (width 0.25) (layer "B.Cu") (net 4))
 (segment (start 167.64 91.44) (end 157.48 101.6) (width 0.25) (layer "F.Cu") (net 3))
 (segment (start 157.48 101.6) (end 125.6382 101.6) (width 0.25) (layer "F.Cu") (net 3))
 (segment (start 111.76 55.88) (end 111.76 73.66) (width 0.25) (layer "F.Cu") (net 3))
 (segment (start 173.1732 85.9068) (end 173.1732 72.446973) (width 0.25) (layer "B.Cu") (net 3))
 (segment (start 173.1732 72.446973) (end 151.526227 50.8) (width 0.25) (layer "B.Cu") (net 3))
 (segment (start 135.7982 57.2418) (end 135.7982 47.955573) (width 0.25) (layer "B.Cu") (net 3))
 (segment (start 168.8182 90.2618) (end 168.8182 88.595573) (width 0.25) (layer "B.Cu") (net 3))
 (segment (start 125.6382 67.4018) (end 125.6382 58.115573) (width 0.25) (layer "B.Cu") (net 3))
 (segment (start 111.76 93.98) (end 111.76 83.82) (width 0.25) (layer "B.Cu") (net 3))
 (segment (start 169.691973 87.7218) (end 171.3582 87.7218) (width 0.25) (layer "B.Cu") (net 3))
 (segment (start 136.671973 47.0818) (end 141.0618 47.0818) (width 0.25) (layer "B.Cu") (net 3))
 (segment (start 111.76 83.82) (end 111.76 73.66) (width 0.25) (layer "B.Cu") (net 3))
 (segment (start 168.8182 88.595573) (end 169.691973 87.7218) (width 0.25) (layer "B.Cu") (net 3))
 (segment (start 119.38 73.66) (end 124.46 68.58) (width 0.25) (layer "B.Cu") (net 3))
 (segment (start 124.46 68.58) (end 125.6382 67.4018) (width 0.25) (layer "B.Cu") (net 3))
 (segment (start 144.78 50.8) (end 142.24 48.26) (width 0.25) (layer "B.Cu") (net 3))
 (segment (start 111.76 73.66) (end 119.38 73.66) (width 0.25) (layer "B.Cu") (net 3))
 (segment (start 134.62 58.42) (end 135.7982 57.2418) (width 0.25) (layer "B.Cu") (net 3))
 (segment (start 141.0618 47.0818) (end 142.24 48.26) (width 0.25) (layer "B.Cu") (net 3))
 (segment (start 151.526227 50.8) (end 144.78 50.8) (width 0.25) (layer "B.Cu") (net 3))
 (segment (start 126.511973 57.2418) (end 133.4418 57.2418) (width 0.25) (layer "B.Cu") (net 3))
 (segment (start 133.4418 57.2418) (end 134.62 58.42) (width 0.25) (layer "B.Cu") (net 3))
 (segment (start 167.64 91.44) (end 168.8182 90.2618) (width 0.25) (layer "B.Cu") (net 3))
 (segment (start 135.7982 47.955573) (end 136.671973 47.0818) (width 0.25) (layer "B.Cu") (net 3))
 (segment (start 171.3582 87.7218) (end 173.1732 85.9068) (width 0.25) (layer "B.Cu") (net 3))
 (segment (start 125.6382 58.115573) (end 126.511973 57.2418) (width 0.25) (layer "B.Cu") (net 3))
 (segment (start 99.06 73.66) (end 106.68 73.66) (width 0.25) (layer "F.Cu") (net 6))
 (segment (start 106.68 68.58) (end 106.68 73.66) (width 0.25) (layer "B.Cu") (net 6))
 (segment (start 127 48.26) (end 106.68 68.58) (width 0.25) (layer "B.Cu") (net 6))
 (segment (start 99.06 83.82) (end 106.68 83.82) (width 0.25) (layer "F.Cu") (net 1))
 (segment (start 104.5932 68.1268) (end 104.5932 81.7332) (width 0.25) (layer "B.Cu") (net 1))
 (segment (start 104.5932 81.7332) (end 106.68 83.82) (width 0.25) (layer "B.Cu") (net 1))
 (segment (start 124.46 48.26) (end 104.5932 68.1268) (width 0.25) (layer "B.Cu") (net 1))
 (segment (start 124.46 101.6) (end 124.46 93.98) (width 0.25) (layer "B.Cu") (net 17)))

